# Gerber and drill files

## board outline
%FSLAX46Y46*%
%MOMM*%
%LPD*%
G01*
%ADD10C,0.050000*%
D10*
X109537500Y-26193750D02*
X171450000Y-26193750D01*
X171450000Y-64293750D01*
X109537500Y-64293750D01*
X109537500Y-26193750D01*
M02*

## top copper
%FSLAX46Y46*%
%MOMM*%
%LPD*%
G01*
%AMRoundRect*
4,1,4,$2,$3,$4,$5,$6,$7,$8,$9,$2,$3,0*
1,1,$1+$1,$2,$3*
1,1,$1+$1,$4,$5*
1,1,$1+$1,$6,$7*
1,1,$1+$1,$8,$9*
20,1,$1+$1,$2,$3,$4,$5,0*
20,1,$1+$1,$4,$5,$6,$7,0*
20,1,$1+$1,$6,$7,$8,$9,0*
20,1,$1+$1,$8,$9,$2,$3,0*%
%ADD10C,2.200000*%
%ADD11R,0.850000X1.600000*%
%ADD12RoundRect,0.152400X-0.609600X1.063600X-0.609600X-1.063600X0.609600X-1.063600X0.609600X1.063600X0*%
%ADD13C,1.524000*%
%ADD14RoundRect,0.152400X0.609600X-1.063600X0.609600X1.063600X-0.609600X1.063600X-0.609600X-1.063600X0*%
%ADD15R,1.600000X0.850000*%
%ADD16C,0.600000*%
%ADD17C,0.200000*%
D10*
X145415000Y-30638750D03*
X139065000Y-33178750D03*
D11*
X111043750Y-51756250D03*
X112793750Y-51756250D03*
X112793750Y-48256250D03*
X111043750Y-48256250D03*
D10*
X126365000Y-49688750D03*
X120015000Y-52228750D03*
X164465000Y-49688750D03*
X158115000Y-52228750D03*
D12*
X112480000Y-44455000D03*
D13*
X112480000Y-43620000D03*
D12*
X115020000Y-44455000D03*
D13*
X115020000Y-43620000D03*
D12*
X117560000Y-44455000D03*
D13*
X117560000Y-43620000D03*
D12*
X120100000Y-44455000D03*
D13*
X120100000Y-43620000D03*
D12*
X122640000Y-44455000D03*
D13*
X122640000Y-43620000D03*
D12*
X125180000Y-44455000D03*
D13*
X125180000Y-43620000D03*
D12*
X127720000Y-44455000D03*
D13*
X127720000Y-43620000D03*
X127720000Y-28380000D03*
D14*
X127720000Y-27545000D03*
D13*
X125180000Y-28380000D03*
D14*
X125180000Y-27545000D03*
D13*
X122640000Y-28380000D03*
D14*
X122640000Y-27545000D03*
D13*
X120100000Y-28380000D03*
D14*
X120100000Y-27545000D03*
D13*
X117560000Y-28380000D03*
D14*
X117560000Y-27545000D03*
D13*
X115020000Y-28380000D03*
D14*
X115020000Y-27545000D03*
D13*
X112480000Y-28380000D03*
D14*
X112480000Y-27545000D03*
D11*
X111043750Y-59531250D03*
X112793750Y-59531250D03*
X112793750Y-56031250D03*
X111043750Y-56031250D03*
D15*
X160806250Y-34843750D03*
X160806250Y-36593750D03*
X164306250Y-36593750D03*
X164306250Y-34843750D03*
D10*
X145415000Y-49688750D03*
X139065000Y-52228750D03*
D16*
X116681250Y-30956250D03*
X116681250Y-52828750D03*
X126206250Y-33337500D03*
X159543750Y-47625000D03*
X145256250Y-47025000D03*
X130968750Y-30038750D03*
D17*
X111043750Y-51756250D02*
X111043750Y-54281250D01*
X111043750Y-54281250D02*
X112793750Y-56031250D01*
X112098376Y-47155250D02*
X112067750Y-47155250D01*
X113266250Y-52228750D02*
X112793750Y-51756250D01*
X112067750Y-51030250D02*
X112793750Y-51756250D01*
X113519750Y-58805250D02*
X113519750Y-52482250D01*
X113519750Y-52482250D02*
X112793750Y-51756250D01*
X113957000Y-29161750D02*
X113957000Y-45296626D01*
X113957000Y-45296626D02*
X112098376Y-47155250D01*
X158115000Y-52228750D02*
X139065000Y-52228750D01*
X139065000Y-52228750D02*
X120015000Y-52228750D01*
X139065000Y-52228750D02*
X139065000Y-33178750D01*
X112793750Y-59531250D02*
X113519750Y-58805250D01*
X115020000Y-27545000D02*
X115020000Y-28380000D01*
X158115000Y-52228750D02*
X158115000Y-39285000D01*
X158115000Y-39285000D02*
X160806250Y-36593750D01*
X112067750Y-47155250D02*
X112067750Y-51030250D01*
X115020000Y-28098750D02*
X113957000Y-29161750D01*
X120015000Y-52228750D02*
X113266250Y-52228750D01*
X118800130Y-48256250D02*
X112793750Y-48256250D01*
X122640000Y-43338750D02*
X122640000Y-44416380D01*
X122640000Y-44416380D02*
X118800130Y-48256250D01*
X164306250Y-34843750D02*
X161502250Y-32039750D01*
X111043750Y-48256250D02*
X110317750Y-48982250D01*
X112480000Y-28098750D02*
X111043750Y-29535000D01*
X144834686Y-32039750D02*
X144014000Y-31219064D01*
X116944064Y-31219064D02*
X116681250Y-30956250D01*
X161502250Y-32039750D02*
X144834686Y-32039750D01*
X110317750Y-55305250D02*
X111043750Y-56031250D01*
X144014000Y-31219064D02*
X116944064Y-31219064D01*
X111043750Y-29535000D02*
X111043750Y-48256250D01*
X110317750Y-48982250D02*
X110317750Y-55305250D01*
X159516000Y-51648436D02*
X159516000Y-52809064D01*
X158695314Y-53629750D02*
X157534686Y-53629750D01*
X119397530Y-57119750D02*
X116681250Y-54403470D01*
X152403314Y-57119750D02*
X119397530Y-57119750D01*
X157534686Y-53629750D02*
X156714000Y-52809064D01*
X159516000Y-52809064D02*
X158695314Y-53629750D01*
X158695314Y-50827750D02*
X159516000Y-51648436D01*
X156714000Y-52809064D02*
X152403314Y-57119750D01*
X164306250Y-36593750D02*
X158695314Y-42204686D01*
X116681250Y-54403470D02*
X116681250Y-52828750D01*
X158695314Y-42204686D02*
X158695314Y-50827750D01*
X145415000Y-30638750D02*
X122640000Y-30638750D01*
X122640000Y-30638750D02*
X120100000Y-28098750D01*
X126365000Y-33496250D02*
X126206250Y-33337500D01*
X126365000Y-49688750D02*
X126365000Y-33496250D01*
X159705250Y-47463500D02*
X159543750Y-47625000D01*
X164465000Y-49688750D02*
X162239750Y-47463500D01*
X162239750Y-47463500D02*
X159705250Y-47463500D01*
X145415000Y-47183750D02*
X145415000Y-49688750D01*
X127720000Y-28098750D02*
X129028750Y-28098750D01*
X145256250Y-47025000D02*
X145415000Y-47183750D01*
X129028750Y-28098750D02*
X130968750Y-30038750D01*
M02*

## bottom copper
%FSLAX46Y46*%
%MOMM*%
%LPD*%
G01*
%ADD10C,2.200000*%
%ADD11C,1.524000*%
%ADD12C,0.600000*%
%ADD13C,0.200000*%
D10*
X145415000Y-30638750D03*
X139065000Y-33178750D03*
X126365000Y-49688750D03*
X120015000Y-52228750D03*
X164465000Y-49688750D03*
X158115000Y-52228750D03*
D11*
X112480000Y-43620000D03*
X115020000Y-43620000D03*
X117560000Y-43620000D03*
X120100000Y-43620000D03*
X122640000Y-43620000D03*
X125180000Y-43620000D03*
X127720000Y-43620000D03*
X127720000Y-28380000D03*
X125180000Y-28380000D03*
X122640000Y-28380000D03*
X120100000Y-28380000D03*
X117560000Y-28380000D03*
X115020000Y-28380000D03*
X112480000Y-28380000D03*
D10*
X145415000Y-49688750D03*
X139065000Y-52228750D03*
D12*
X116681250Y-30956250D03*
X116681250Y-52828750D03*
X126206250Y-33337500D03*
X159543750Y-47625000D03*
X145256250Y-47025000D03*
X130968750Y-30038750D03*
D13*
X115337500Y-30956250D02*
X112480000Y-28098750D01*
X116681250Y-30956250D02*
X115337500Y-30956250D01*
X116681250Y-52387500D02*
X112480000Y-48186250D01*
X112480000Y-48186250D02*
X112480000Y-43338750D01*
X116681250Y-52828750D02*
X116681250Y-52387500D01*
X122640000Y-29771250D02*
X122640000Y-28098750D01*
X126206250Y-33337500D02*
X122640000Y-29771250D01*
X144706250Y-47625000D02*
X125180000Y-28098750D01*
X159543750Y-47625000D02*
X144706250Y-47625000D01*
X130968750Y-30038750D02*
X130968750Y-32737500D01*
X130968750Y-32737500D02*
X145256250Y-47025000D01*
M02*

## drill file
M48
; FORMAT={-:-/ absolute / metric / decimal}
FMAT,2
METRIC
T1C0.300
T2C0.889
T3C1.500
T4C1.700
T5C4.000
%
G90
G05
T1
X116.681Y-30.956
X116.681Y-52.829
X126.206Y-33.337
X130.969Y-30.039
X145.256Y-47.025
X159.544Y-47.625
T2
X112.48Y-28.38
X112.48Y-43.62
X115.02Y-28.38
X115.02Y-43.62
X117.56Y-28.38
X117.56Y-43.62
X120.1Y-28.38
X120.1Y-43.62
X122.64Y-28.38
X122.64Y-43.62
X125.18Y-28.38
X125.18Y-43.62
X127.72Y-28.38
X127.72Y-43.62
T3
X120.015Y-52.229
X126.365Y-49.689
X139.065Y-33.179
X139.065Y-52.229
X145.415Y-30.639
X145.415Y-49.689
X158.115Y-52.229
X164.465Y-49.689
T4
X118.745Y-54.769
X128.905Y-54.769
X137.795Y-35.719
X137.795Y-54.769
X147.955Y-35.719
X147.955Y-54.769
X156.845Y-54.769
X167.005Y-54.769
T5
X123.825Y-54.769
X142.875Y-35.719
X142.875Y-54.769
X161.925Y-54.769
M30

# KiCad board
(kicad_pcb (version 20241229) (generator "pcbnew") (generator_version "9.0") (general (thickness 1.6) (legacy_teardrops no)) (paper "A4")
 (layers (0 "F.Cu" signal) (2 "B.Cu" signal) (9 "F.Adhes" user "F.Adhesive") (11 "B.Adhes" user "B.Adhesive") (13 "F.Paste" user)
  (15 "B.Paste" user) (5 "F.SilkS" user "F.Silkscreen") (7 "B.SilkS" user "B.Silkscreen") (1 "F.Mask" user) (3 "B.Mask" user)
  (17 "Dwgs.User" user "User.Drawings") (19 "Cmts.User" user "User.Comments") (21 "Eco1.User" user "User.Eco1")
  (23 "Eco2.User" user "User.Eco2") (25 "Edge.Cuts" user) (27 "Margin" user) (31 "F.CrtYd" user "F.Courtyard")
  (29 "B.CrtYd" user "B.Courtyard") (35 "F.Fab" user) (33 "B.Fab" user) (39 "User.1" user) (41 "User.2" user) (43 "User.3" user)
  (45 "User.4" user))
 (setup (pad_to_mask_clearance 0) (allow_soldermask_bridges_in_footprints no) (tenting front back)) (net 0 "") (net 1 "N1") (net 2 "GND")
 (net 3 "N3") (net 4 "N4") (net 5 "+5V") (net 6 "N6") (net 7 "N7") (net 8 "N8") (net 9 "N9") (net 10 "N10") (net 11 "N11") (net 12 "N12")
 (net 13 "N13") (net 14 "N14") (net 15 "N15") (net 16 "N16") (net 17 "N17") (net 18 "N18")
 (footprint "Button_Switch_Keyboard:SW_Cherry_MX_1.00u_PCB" (layer "F.Cu") (at 145.415 30.63875)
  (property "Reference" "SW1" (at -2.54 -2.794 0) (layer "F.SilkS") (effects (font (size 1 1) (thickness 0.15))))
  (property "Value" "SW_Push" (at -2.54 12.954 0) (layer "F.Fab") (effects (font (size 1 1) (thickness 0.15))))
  (pad "" np_thru_hole circle (at -7.62 5.08) (size 1.7 1.7) (drill 1.7) (layers "*.Cu" "*.Mask"))
  (pad "" np_thru_hole circle (at -2.54 5.08) (size 4 4) (drill 4) (layers "*.Cu" "*.Mask"))
  (pad "" np_thru_hole circle (at 2.54 5.08) (size 1.7 1.7) (drill 1.7) (layers "*.Cu" "*.Mask"))
  (pad "1" thru_hole circle (at 0 0) (size 2.2 2.2) (drill 1.5) (layers "*.Cu" "*.Mask") (remove_unused_layers no) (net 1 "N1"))
  (pad "2" thru_hole circle (at -6.35 2.54) (size 2.2 2.2) (drill 1.5) (layers "*.Cu" "*.Mask") (remove_unused_layers no) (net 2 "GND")))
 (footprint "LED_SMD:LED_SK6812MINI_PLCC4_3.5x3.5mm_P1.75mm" (layer "F.Cu") (at 111.91875 50.00625 90)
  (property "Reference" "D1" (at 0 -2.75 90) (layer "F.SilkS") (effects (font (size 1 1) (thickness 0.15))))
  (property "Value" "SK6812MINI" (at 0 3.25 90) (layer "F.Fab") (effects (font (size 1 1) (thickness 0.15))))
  (pad "1" smd rect (at -1.75 -0.875 90) (size 1.6 0.85) (layers "F.Cu" "F.Mask" "F.Paste") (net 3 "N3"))
  (pad "2" smd rect (at -1.75 0.875 90) (size 1.6 0.85) (layers "F.Cu" "F.Mask" "F.Paste") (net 2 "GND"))
  (pad "3" smd rect (at 1.75 0.875 90) (size 1.6 0.85) (layers "F.Cu" "F.Mask" "F.Paste") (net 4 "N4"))
  (pad "4" smd rect (at 1.75 -0.875 90) (size 1.6 0.85) (layers "F.Cu" "F.Mask" "F.Paste") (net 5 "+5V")))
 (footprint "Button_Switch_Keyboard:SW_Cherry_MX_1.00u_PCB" (layer "F.Cu") (at 126.365 49.68875)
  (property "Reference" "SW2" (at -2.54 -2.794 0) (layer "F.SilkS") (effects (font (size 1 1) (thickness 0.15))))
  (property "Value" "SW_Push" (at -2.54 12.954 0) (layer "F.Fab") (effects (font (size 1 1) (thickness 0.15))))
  (pad "" np_thru_hole circle (at -7.62 5.08) (size 1.7 1.7) (drill 1.7) (layers "*.Cu" "*.Mask"))
  (pad "" np_thru_hole circle (at -2.54 5.08) (size 4 4) (drill 4) (layers "*.Cu" "*.Mask"))
  (pad "" np_thru_hole circle (at 2.54 5.08) (size 1.7 1.7) (drill 1.7) (layers "*.Cu" "*.Mask"))
  (pad "1" thru_hole circle (at 0 0) (size 2.2 2.2) (drill 1.5) (layers "*.Cu" "*.Mask") (remove_unused_layers no) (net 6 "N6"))
  (pad "2" thru_hole circle (at -6.35 2.54) (size 2.2 2.2) (drill 1.5) (layers "*.Cu" "*.Mask") (remove_unused_layers no) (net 2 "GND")))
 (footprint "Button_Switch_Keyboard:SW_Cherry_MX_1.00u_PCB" (layer "F.Cu") (at 164.465 49.68875)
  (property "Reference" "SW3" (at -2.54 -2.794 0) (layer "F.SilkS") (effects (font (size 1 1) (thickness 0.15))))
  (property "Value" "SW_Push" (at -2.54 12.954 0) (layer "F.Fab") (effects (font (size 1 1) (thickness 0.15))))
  (pad "" np_thru_hole circle (at -7.62 5.08) (size 1.7 1.7) (drill 1.7) (layers "*.Cu" "*.Mask"))
  (pad "" np_thru_hole circle (at -2.54 5.08) (size 4 4) (drill 4) (layers "*.Cu" "*.Mask"))
  (pad "" np_thru_hole circle (at 2.54 5.08) (size 1.7 1.7) (drill 1.7) (layers "*.Cu" "*.Mask"))
  (pad "1" thru_hole circle (at 0 0) (size 2.2 2.2) (drill 1.5) (layers "*.Cu" "*.Mask") (remove_unused_layers no) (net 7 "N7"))
  (pad "2" thru_hole circle (at -6.35 2.54) (size 2.2 2.2) (drill 1.5) (layers "*.Cu" "*.Mask") (remove_unused_layers no) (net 2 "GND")))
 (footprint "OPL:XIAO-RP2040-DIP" (layer "F.Cu") (at 120.1 36 90)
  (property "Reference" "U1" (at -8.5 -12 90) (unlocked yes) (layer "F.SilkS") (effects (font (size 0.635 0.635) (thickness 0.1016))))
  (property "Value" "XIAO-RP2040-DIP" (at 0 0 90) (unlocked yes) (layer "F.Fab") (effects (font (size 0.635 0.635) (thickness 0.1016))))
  (pad "1" smd roundrect (at -8.455 -7.62 270) (size 2.432 1.524) (layers "F.Cu" "F.Mask") (roundrect_rratio 0.1) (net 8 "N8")
   (thermal_bridge_angle 45))
  (pad "1" thru_hole circle (at -7.62 -7.62 270) (size 1.524 1.524) (drill 0.889) (layers "*.Cu" "*.Mask") (remove_unused_layers no)
   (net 8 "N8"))
  (pad "2" smd roundrect (at -8.455 -5.08 270) (size 2.432 1.524) (layers "F.Cu" "F.Mask") (roundrect_rratio 0.1) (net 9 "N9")
   (thermal_bridge_angle 45))
  (pad "2" thru_hole circle (at -7.62 -5.08 270) (size 1.524 1.524) (drill 0.889) (layers "*.Cu" "*.Mask") (remove_unused_layers no)
   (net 9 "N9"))
  (pad "3" smd roundrect (at -8.455 -2.54 270) (size 2.432 1.524) (layers "F.Cu" "F.Mask") (roundrect_rratio 0.1) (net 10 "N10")
   (thermal_bridge_angle 45))
  (pad "3" thru_hole circle (at -7.62 -2.54 270) (size 1.524 1.524) (drill 0.889) (layers "*.Cu" "*.Mask") (remove_unused_layers no)
   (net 10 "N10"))
  (pad "4" smd roundrect (at -8.455 0 270) (size 2.432 1.524) (layers "F.Cu" "F.Mask") (roundrect_rratio 0.1) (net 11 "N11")
   (thermal_bridge_angle 45))
  (pad "4" thru_hole circle (at -7.62 0 270) (size 1.524 1.524) (drill 0.889) (layers "*.Cu" "*.Mask") (remove_unused_layers no)
   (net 11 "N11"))
  (pad "5" smd roundrect (at -8.455 2.54 270) (size 2.432 1.524) (layers "F.Cu" "F.Mask") (roundrect_rratio 0.1) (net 4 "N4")
   (thermal_bridge_angle 45))
  (pad "5" thru_hole circle (at -7.62 2.54 270) (size 1.524 1.524) (drill 0.889) (layers "*.Cu" "*.Mask") (remove_unused_layers no)
   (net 4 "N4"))
  (pad "6" smd roundrect (at -8.455 5.08 270) (size 2.432 1.524) (layers "F.Cu" "F.Mask") (roundrect_rratio 0.1) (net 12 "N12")
   (thermal_bridge_angle 45))
  (pad "6" thru_hole circle (at -7.62 5.08 270) (size 1.524 1.524) (drill 0.889) (layers "*.Cu" "*.Mask") (remove_unused_layers no)
   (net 12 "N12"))
  (pad "7" smd roundrect (at -8.455 7.62 270) (size 2.432 1.524) (layers "F.Cu" "F.Mask") (roundrect_rratio 0.1) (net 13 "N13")
   (thermal_bridge_angle 45))
  (pad "7" thru_hole circle (at -7.62 7.62 270) (size 1.524 1.524) (drill 0.889) (layers "*.Cu" "*.Mask") (remove_unused_layers no)
   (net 13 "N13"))
  (pad "8" thru_hole circle (at 7.62 7.62 90) (size 1.524 1.524) (drill 0.889) (layers "*.Cu" "*.Mask") (remove_unused_layers no)
   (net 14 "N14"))
  (pad "8" smd roundrect (at 8.455 7.62 90) (size 2.432 1.524) (layers "F.Cu" "F.Mask") (roundrect_rratio 0.1) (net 14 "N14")
   (thermal_bridge_angle 45))
  (pad "9" thru_hole circle (at 7.62 5.08 90) (size 1.524 1.524) (drill 0.889) (layers "*.Cu" "*.Mask") (remove_unused_layers no)
   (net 7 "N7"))
  (pad "9" smd roundrect (at 8.455 5.08 90) (size 2.432 1.524) (layers "F.Cu" "F.Mask") (roundrect_rratio 0.1) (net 7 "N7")
   (thermal_bridge_angle 45))
  (pad "10" thru_hole circle (at 7.62 2.54 90) (size 1.524 1.524) (drill 0.889) (layers "*.Cu" "*.Mask") (remove_unused_layers no)
   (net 6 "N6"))
  (pad "10" smd roundrect (at 8.455 2.54 90) (size 2.432 1.524) (layers "F.Cu" "F.Mask") (roundrect_rratio 0.1) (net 6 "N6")
   (thermal_bridge_angle 45))
  (pad "11" thru_hole circle (at 7.62 0 90) (size 1.524 1.524) (drill 0.889) (layers "*.Cu" "*.Mask") (remove_unused_layers no) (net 1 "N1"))
  (pad "11" smd roundrect (at 8.455 0 90) (size 2.432 1.524) (layers "F.Cu" "F.Mask") (roundrect_rratio 0.1) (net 1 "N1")
   (thermal_bridge_angle 45))
  (pad "12" thru_hole circle (at 7.62 -2.54 90) (size 1.524 1.524) (drill 0.889) (layers "*.Cu" "*.Mask") (remove_unused_layers no)
   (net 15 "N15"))
  (pad "12" smd roundrect (at 8.455 -2.54 90) (size 2.432 1.524) (layers "F.Cu" "F.Mask") (roundrect_rratio 0.1) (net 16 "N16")
   (thermal_bridge_angle 45))
  (pad "13" thru_hole circle (at 7.62 -5.08 90) (size 1.524 1.524) (drill 0.889) (layers "*.Cu" "*.Mask") (remove_unused_layers no)
   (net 2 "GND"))
  (pad "13" smd roundrect (at 8.455 -5.08 90) (size 2.432 1.524) (layers "F.Cu" "F.Mask") (roundrect_rratio 0.1) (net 2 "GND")
   (thermal_bridge_angle 45))
  (pad "14" thru_hole circle (at 7.62 -7.62 90) (size 1.524 1.524) (drill 0.889) (layers "*.Cu" "*.Mask") (remove_unused_layers no)
   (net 5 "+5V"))
  (pad "14" smd roundrect (at 8.455 -7.62 90) (size 2.432 1.524) (layers "F.Cu" "F.Mask") (roundrect_rratio 0.1) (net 5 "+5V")
   (thermal_bridge_angle 45)))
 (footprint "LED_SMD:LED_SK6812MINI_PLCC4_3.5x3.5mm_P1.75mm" (layer "F.Cu") (at 111.91875 57.78125 90)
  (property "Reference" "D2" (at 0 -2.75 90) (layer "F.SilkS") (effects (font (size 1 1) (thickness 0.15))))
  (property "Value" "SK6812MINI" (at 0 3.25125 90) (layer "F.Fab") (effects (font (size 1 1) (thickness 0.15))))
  (pad "1" smd rect (at -1.75 -0.875 90) (size 1.6 0.85) (layers "F.Cu" "F.Mask" "F.Paste") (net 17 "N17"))
  (pad "2" smd rect (at -1.75 0.875 90) (size 1.6 0.85) (layers "F.Cu" "F.Mask" "F.Paste") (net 2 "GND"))
  (pad "3" smd rect (at 1.75 0.875 90) (size 1.6 0.85) (layers "F.Cu" "F.Mask" "F.Paste") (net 3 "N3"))
  (pad "4" smd rect (at 1.75 -0.875 90) (size 1.6 0.85) (layers "F.Cu" "F.Mask" "F.Paste") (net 5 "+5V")))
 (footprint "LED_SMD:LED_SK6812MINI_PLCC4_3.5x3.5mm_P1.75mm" (layer "F.Cu") (at 162.55625 35.71875)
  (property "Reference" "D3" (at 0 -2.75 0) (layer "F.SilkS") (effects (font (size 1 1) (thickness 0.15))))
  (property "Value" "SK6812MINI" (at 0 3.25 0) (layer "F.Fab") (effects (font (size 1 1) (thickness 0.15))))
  (pad "1" smd rect (at -1.75 -0.875) (size 1.6 0.85) (layers "F.Cu" "F.Mask" "F.Paste") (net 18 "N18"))
  (pad "2" smd rect (at -1.75 0.875) (size 1.6 0.85) (layers "F.Cu" "F.Mask" "F.Paste") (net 2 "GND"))
  (pad "3" smd rect (at 1.75 0.875) (size 1.6 0.85) (layers "F.Cu" "F.Mask" "F.Paste") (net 8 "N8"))
  (pad "4" smd rect (at 1.75 -0.875) (size 1.6 0.85) (layers "F.Cu" "F.Mask" "F.Paste") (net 5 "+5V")))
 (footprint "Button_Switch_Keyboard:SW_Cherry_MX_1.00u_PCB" (layer "F.Cu") (at 145.415 49.68875)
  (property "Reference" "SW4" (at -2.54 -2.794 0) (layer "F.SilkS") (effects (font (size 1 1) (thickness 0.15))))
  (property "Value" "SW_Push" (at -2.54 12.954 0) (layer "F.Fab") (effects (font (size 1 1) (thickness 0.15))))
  (pad "" np_thru_hole circle (at -7.62 5.08) (size 1.7 1.7) (drill 1.7) (layers "*.Cu" "*.Mask"))
  (pad "" np_thru_hole circle (at -2.54 5.08) (size 4 4) (drill 4) (layers "*.Cu" "*.Mask"))
  (pad "" np_thru_hole circle (at 2.54 5.08) (size 1.7 1.7) (drill 1.7) (layers "*.Cu" "*.Mask"))
  (pad "1" thru_hole circle (at 0 0) (size 2.2 2.2) (drill 1.5) (layers "*.Cu" "*.Mask") (remove_unused_layers no) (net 14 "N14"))
  (pad "2" thru_hole circle (at -6.35 2.54) (size 2.2 2.2) (drill 1.5) (layers "*.Cu" "*.Mask") (remove_unused_layers no) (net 2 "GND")))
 (gr_rect (start 109.5375 26.19375) (end 171.45 64.29375) (stroke (width 0.05) (type default)) (fill no) (layer "Edge.Cuts"))
 (segment (start 111.04375 51.75625) (end 111.04375 54.28125) (width 0.2) (layer "F.Cu") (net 3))
 (segment (start 111.04375 54.28125) (end 112.79375 56.03125) (width 0.2) (layer "F.Cu") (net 3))
 (segment (start 112.098376 47.15525) (end 112.06775 47.15525) (width 0.2) (layer "F.Cu") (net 2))
 (segment (start 113.26625 52.22875) (end 112.79375 51.75625) (width 0.2) (layer "F.Cu") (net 2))
 (segment (start 112.06775 51.03025) (end 112.79375 51.75625) (width 0.2) (layer "F.Cu") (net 2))
 (segment (start 113.51975 58.80525) (end 113.51975 52.48225) (width 0.2) (layer "F.Cu") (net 2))
 (segment (start 113.51975 52.48225) (end 112.79375 51.75625) (width 0.2) (layer "F.Cu") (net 2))
 (segment (start 113.957 29.16175) (end 113.957 45.296626) (width 0.2) (layer "F.Cu") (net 2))
 (segment (start 113.957 45.296626) (end 112.098376 47.15525) (width 0.2) (layer "F.Cu") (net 2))
 (segment (start 158.115 52.22875) (end 139.065 52.22875) (width 0.2) (layer "F.Cu") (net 2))
 (segment (start 139.065 52.22875) (end 120.015 52.22875) (width 0.2) (layer "F.Cu") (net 2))
 (segment (start 139.065 52.22875) (end 139.065 33.17875) (width 0.2) (layer "F.Cu") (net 2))
 (segment (start 112.79375 59.53125) (end 113.51975 58.80525) (width 0.2) (layer "F.Cu") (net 2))
 (segment (start 115.02 27.545) (end 115.02 28.38) (width 0.2) (layer "F.Cu") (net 2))
 (segment (start 158.115 52.22875) (end 158.115 39.285) (width 0.2) (layer "F.Cu") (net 2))
 (segment (start 158.115 39.285) (end 160.80625 36.59375) (width 0.2) (layer "F.Cu") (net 2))
 (segment (start 112.06775 47.15525) (end 112.06775 51.03025) (width 0.2) (layer "F.Cu") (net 2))
 (segment (start 115.02 28.09875) (end 113.957 29.16175) (width 0.2) (layer "F.Cu") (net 2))
 (segment (start 120.015 52.22875) (end 113.26625 52.22875) (width 0.2) (layer "F.Cu") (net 2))
 (segment (start 118.80013 48.25625) (end 112.79375 48.25625) (width 0.2) (layer "F.Cu") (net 4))
 (segment (start 122.64 43.33875) (end 122.64 44.41638) (width 0.2) (layer "F.Cu") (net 4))
 (segment (start 122.64 44.41638) (end 118.80013 48.25625) (width 0.2) (layer "F.Cu") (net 4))
 (segment (start 164.30625 34.84375) (end 161.50225 32.03975) (width 0.2) (layer "F.Cu") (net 5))
 (segment (start 111.04375 48.25625) (end 110.31775 48.98225) (width 0.2) (layer "F.Cu") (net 5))
 (segment (start 112.48 28.09875) (end 111.04375 29.535) (width 0.2) (layer "F.Cu") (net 5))
 (segment (start 144.834686 32.03975) (end 144.014 31.219064) (width 0.2) (layer "F.Cu") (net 5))
 (segment (start 116.944064 31.219064) (end 116.68125 30.95625) (width 0.2) (layer "F.Cu") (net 5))
 (segment (start 161.50225 32.03975) (end 144.834686 32.03975) (width 0.2) (layer "F.Cu") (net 5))
 (segment (start 110.31775 55.30525) (end 111.04375 56.03125) (width 0.2) (layer "F.Cu") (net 5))
 (segment (start 144.014 31.219064) (end 116.944064 31.219064) (width 0.2) (layer "F.Cu") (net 5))
 (segment (start 111.04375 29.535) (end 111.04375 48.25625) (width 0.2) (layer "F.Cu") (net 5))
 (segment (start 110.31775 48.98225) (end 110.31775 55.30525) (width 0.2) (layer "F.Cu") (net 5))
 (via (at 116.68125 30.95625) (size 0.6) (drill 0.3) (layers "F.Cu" "B.Cu") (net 5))
 (segment (start 115.3375 30.95625) (end 112.48 28.09875) (width 0.2) (layer "B.Cu") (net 5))
 (segment (start 116.68125 30.95625) (end 115.3375 30.95625) (width 0.2) (layer "B.Cu") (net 5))
 (segment (start 159.516 51.648436) (end 159.516 52.809064) (width 0.2) (layer "F.Cu") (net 8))
 (segment (start 158.695314 53.62975) (end 157.534686 53.62975) (width 0.2) (layer "F.Cu") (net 8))
 (segment (start 119.39753 57.11975) (end 116.68125 54.40347) (width 0.2) (layer "F.Cu") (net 8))
 (segment (start 152.403314 57.11975) (end 119.39753 57.11975) (width 0.2) (layer "F.Cu") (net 8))
 (segment (start 157.534686 53.62975) (end 156.714 52.809064) (width 0.2) (layer "F.Cu") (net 8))
 (segment (start 159.516 52.809064) (end 158.695314 53.62975) (width 0.2) (layer "F.Cu") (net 8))
 (segment (start 158.695314 50.82775) (end 159.516 51.648436) (width 0.2) (layer "F.Cu") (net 8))
 (segment (start 156.714 52.809064) (end 152.403314 57.11975) (width 0.2) (layer "F.Cu") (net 8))
 (segment (start 164.30625 36.59375) (end 158.695314 42.204686) (width 0.2) (layer "F.Cu") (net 8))
 (segment (start 116.68125 54.40347) (end 116.68125 52.82875) (width 0.2) (layer "F.Cu") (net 8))
 (segment (start 158.695314 42.204686) (end 158.695314 50.82775) (width 0.2) (layer "F.Cu") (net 8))
 (via (at 116.68125 52.82875) (size 0.6) (drill 0.3) (layers "F.Cu" "B.Cu") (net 8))
 (segment (start 116.68125 52.3875) (end 112.48 48.18625) (width 0.2) (layer "B.Cu") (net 8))
 (segment (start 112.48 48.18625) (end 112.48 43.33875) (width 0.2) (layer "B.Cu") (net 8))
 (segment (start 116.68125 52.82875) (end 116.68125 52.3875) (width 0.2) (layer "B.Cu") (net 8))
 (segment (start 145.415 30.63875) (end 122.64 30.63875) (width 0.2) (layer "F.Cu") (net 1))
 (segment (start 122.64 30.63875) (end 120.1 28.09875) (width 0.2) (layer "F.Cu") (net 1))
 (segment (start 126.365 33.49625) (end 126.20625 33.3375) (width 0.2) (layer "F.Cu") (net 6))
 (segment (start 126.365 49.68875) (end 126.365 33.49625) (width 0.2) (layer "F.Cu") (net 6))
 (via (at 126.20625 33.3375) (size 0.6) (drill 0.3) (layers "F.Cu" "B.Cu") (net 6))
 (segment (start 122.64 29.77125) (end 122.64 28.09875) (width 0.2) (layer "B.Cu") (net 6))
 (segment (start 126.20625 33.3375) (end 122.64 29.77125) (width 0.2) (layer "B.Cu") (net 6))
 (segment (start 159.70525 47.4635) (end 159.54375 47.625) (width 0.2) (layer "F.Cu") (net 7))
 (segment (start 164.465 49.68875) (end 162.23975 47.4635) (width 0.2) (layer "F.Cu") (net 7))
 (segment (start 162.23975 47.4635) (end 159.70525 47.4635) (width 0.2) (layer "F.Cu") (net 7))
 (via (at 159.54375 47.625) (size 0.6) (drill 0.3) (layers "F.Cu" "B.Cu") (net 7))
 (segment (start 144.70625 47.625) (end 125.18 28.09875) (width 0.2) (layer "B.Cu") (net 7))
 (segment (start 159.54375 47.625) (end 144.70625 47.625) (width 0.2) (layer "B.Cu") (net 7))
 (segment (start 145.415 47.18375) (end 145.415 49.68875) (width 0.2) (layer "F.Cu") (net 14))
 (segment (start 127.72 28.09875) (end 129.02875 28.09875) (width 0.2) (layer "F.Cu") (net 14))
 (segment (start 145.25625 47.025) (end 145.415 47.18375) (width 0.2) (layer "F.Cu") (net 14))
 (segment (start 129.02875 28.09875) (end 130.96875 30.03875) (width 0.2) (layer "F.Cu") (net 14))
 (via (at 145.25625 47.025) (size 0.6) (drill 0.3) (layers "F.Cu" "B.Cu") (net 14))
 (via (at 130.96875 30.03875) (size 0.6) (drill 0.3) (layers "F.Cu" "B.Cu") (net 14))
 (segment (start 130.96875 30.03875) (end 130.96875 32.7375) (width 0.2) (layer "B.Cu") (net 14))
 (segment (start 130.96875 32.7375) (end 145.25625 47.025) (width 0.2) (layer "B.Cu") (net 14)))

